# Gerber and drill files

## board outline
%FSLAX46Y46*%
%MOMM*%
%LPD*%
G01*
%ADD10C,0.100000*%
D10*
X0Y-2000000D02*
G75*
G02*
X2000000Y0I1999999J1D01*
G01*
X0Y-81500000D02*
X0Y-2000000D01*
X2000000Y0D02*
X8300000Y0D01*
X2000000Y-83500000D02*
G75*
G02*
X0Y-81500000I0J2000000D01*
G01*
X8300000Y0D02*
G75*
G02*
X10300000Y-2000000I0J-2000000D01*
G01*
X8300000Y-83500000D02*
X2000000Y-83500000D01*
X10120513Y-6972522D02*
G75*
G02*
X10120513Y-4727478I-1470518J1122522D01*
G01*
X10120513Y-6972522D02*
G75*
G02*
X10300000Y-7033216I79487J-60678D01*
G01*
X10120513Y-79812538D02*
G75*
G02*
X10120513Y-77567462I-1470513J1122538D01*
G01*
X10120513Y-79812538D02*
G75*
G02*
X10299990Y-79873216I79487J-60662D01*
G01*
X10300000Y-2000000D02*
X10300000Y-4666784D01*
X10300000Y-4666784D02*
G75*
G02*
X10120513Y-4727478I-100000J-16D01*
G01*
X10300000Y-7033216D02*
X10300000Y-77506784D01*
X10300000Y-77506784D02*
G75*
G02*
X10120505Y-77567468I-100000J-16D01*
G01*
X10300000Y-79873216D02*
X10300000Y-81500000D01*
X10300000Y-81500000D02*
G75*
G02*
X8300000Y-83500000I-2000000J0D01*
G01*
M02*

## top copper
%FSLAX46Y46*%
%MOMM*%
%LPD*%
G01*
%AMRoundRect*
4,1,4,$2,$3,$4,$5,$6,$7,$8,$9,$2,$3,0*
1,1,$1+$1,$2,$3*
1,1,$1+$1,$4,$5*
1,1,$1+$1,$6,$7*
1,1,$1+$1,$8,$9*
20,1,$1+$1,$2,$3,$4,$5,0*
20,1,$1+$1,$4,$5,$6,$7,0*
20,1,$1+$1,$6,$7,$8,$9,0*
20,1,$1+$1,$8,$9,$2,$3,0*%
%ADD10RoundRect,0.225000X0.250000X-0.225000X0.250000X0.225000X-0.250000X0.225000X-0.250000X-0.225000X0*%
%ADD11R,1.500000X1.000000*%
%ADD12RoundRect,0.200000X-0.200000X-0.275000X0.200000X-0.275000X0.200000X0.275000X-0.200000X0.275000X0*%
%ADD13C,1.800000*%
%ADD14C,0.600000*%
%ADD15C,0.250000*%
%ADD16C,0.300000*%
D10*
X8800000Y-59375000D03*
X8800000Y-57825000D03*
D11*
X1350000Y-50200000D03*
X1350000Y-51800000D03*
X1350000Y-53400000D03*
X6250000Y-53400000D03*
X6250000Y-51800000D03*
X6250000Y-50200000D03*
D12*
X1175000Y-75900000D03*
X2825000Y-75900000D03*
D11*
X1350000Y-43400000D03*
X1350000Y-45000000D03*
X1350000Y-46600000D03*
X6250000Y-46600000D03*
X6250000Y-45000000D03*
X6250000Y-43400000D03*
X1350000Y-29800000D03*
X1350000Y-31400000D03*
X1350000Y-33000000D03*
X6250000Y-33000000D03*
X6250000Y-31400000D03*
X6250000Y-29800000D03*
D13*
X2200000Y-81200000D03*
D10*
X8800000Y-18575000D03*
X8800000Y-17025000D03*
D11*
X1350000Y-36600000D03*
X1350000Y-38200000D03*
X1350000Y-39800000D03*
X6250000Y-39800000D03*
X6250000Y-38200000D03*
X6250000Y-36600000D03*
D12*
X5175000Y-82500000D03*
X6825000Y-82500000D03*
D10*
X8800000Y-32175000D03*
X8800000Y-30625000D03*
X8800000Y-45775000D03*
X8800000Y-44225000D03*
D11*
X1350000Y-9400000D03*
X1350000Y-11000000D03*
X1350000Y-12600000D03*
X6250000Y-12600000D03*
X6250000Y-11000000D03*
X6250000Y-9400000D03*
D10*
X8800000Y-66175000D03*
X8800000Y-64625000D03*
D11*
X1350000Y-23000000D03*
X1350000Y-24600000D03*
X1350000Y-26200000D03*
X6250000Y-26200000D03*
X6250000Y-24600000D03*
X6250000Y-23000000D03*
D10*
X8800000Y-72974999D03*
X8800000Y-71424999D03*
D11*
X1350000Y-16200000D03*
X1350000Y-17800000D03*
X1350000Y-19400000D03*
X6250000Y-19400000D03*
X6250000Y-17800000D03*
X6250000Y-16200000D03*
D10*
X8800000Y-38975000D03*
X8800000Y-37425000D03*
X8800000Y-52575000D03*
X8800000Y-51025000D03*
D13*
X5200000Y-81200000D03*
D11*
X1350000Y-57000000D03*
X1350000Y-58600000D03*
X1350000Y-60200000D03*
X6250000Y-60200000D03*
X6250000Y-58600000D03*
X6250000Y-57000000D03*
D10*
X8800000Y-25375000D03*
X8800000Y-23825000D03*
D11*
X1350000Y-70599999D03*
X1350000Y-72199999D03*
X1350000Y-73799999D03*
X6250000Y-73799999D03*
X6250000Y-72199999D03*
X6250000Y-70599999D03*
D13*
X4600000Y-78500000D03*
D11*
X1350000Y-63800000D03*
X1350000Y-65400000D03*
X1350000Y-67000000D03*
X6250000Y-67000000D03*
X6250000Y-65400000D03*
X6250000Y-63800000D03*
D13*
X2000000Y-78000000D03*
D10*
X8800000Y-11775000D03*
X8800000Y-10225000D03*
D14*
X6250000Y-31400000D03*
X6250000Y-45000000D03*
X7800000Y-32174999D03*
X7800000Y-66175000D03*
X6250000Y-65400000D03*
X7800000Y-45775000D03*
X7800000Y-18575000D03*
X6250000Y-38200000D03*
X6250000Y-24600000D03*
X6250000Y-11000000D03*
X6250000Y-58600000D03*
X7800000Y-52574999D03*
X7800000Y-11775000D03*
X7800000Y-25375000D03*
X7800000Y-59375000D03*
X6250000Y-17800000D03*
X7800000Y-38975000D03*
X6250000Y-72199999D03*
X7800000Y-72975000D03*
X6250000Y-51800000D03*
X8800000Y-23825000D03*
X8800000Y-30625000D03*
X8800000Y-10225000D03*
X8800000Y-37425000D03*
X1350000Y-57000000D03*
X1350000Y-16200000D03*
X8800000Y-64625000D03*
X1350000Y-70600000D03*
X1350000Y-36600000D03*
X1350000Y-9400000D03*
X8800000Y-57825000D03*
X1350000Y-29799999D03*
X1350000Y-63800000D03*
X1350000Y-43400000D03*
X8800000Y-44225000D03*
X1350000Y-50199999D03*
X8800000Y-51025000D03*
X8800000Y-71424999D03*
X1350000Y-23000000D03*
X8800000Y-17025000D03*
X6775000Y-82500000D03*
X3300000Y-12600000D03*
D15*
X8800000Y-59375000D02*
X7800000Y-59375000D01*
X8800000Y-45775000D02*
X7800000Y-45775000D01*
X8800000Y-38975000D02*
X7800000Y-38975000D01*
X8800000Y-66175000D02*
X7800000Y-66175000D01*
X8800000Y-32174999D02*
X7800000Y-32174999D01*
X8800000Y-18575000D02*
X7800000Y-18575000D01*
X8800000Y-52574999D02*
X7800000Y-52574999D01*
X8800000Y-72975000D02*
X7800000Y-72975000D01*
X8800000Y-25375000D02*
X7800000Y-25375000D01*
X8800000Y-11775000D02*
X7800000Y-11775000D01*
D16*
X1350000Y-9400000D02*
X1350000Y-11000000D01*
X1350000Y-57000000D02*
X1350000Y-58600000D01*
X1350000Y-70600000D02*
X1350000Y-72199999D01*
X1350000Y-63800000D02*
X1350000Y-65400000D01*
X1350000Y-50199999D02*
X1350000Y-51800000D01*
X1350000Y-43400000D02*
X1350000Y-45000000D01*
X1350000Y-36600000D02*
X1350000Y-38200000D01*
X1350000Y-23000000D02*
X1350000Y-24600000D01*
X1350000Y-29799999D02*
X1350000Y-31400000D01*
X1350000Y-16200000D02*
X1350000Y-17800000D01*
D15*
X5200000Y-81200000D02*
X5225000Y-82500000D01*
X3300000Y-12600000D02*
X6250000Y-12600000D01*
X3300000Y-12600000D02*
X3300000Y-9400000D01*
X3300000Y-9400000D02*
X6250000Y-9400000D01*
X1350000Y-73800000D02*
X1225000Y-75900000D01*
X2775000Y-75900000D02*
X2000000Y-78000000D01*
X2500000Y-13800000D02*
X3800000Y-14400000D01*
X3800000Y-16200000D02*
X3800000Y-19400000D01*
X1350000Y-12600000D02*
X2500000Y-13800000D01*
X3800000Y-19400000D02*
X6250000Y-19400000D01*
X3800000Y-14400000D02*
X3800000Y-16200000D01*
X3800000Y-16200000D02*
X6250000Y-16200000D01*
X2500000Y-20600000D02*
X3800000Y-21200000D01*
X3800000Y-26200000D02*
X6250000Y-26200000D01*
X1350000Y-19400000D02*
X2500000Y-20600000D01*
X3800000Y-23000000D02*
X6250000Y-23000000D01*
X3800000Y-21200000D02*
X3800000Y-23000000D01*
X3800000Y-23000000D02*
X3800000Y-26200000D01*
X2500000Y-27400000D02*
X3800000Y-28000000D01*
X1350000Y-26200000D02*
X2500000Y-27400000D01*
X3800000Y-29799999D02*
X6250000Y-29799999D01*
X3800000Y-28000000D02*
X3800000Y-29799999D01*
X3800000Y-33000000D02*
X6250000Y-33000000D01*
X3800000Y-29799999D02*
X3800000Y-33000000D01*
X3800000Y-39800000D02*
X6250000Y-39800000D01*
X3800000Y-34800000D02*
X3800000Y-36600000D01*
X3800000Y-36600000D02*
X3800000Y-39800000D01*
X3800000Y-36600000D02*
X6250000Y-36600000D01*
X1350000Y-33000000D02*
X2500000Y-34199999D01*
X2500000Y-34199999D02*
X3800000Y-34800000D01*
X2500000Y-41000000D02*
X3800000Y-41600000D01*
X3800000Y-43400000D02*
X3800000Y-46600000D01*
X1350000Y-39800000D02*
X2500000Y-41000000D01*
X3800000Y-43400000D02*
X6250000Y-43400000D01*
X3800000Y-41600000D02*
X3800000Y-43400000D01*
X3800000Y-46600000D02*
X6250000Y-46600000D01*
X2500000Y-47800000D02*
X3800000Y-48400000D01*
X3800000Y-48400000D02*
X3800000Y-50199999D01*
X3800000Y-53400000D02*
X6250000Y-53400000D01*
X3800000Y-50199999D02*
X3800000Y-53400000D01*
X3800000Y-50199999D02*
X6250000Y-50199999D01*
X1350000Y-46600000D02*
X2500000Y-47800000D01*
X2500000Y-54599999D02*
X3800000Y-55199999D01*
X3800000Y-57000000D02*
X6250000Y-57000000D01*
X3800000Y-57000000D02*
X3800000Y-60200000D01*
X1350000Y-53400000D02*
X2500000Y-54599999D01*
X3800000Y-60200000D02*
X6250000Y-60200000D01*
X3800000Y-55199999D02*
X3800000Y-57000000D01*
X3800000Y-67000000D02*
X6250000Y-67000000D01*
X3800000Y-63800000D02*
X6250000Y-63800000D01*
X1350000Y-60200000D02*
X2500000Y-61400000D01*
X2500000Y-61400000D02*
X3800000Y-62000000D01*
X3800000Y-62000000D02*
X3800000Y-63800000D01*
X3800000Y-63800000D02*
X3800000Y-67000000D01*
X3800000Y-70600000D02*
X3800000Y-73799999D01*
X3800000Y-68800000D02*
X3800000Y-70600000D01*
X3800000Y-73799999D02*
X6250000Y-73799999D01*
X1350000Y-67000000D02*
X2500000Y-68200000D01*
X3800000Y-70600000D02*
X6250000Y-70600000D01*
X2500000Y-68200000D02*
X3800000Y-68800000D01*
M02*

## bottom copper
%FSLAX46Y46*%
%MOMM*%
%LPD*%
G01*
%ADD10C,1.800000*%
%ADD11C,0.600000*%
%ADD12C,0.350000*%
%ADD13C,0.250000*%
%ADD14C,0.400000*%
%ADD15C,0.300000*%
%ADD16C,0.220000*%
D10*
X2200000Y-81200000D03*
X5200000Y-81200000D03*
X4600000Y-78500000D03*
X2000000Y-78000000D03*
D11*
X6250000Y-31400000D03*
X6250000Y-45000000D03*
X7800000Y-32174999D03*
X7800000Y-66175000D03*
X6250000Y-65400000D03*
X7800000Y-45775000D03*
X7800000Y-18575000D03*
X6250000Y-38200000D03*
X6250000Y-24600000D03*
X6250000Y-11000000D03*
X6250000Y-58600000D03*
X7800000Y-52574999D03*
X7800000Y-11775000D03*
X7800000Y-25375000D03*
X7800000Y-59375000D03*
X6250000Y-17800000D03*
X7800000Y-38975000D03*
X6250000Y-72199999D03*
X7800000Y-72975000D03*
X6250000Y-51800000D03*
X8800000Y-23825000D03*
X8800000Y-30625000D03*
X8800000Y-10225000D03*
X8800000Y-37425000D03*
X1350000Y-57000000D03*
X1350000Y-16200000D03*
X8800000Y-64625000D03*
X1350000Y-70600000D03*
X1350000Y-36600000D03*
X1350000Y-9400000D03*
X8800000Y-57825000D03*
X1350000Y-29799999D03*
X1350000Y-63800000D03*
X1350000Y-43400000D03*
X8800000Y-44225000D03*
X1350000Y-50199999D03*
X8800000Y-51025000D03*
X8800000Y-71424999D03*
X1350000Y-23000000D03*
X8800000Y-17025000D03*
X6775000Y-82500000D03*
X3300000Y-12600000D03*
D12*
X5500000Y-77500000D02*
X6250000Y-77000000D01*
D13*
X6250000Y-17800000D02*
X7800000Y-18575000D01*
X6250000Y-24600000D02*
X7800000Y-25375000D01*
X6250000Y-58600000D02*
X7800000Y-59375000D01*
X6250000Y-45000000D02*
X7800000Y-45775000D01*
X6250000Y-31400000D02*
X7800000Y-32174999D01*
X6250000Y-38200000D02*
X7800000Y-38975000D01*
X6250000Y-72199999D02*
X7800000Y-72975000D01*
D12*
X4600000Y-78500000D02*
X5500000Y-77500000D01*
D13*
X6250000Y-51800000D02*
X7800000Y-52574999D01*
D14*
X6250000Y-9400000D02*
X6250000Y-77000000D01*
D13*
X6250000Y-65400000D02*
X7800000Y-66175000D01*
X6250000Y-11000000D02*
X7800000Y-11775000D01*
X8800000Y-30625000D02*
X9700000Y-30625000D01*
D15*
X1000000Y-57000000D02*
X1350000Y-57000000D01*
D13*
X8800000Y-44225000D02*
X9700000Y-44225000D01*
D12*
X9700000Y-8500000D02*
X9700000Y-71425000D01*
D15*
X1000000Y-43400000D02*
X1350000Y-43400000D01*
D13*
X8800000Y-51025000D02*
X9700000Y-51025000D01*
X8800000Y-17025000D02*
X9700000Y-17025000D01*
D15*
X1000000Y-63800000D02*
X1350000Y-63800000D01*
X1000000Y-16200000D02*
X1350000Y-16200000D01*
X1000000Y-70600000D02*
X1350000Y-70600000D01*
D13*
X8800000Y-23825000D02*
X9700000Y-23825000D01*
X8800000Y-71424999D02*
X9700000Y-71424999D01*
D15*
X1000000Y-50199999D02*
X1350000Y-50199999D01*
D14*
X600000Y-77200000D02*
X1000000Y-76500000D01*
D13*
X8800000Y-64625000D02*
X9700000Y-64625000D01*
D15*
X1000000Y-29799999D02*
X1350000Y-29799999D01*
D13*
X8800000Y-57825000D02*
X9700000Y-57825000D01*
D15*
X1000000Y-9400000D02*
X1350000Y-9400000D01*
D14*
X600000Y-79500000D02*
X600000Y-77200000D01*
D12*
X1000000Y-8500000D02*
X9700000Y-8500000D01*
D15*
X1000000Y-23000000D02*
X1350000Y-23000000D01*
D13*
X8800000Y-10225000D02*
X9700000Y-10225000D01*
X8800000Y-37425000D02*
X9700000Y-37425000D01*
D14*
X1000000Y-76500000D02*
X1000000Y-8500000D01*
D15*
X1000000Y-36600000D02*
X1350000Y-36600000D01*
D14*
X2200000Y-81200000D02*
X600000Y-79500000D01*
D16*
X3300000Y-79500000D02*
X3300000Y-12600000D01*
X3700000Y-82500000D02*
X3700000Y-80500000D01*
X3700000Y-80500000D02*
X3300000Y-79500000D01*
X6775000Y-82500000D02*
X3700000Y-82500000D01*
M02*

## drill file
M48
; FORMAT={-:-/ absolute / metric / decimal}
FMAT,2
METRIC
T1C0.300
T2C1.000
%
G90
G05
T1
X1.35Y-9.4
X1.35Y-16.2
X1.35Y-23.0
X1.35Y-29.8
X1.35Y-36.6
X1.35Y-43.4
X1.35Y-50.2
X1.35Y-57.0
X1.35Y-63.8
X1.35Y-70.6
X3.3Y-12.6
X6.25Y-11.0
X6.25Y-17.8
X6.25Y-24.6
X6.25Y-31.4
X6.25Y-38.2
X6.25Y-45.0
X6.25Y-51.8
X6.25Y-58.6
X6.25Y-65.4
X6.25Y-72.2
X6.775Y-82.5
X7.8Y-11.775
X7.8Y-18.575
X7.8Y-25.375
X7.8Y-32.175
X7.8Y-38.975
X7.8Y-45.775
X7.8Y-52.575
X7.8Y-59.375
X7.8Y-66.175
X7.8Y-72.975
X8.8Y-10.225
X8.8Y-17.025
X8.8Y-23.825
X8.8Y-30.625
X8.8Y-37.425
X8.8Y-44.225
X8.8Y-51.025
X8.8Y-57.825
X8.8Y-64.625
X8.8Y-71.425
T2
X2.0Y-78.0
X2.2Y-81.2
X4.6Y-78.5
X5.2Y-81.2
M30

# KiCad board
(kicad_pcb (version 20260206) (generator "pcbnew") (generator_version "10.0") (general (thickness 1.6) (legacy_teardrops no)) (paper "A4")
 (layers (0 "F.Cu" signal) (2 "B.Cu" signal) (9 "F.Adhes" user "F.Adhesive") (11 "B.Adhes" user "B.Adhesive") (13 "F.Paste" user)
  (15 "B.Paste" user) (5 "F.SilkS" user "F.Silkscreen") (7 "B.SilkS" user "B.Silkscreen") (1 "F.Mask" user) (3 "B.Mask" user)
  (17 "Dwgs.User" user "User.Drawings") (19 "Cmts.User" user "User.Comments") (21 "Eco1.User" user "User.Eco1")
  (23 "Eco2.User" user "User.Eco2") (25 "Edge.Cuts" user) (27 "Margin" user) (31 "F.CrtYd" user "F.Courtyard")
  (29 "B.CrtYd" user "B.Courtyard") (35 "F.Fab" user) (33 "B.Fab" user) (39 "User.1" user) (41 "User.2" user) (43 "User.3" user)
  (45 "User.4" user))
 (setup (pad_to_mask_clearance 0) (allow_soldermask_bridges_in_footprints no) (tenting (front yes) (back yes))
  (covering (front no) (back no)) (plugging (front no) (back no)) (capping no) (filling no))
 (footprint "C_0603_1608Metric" (layer "F.Cu") (at 8.8 58.6 90)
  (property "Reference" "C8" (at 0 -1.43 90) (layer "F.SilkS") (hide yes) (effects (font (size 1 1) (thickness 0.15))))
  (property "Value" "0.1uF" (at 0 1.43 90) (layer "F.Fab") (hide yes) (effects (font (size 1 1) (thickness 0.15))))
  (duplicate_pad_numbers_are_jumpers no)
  (pad "1" smd roundrect (at -0.775 0 90) (size 0.9 0.95) (layers "F.Cu" "F.Mask" "F.Paste") (roundrect_rratio 0.25) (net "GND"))
  (pad "2" smd roundrect (at 0.775 0 90) (size 0.9 0.95) (layers "F.Cu" "F.Mask" "F.Paste") (roundrect_rratio 0.25) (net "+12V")))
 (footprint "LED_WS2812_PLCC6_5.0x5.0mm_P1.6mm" (layer "F.Cu") (at 3.8 51.8)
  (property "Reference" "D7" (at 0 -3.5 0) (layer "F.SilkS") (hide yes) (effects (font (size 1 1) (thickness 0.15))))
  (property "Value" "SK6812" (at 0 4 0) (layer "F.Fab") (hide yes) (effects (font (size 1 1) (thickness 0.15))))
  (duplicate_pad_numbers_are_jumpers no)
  (pad "1" smd rect (at -2.45 -1.6) (size 1.5 1) (layers "F.Cu" "F.Mask" "F.Paste") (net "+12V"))
  (pad "2" smd rect (at -2.45 0) (size 1.5 1) (layers "F.Cu" "F.Mask" "F.Paste") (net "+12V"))
  (pad "3" smd rect (at -2.45 1.6) (size 1.5 1) (layers "F.Cu" "F.Mask" "F.Paste") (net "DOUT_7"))
  (pad "4" smd rect (at 2.45 1.6) (size 1.5 1) (layers "F.Cu" "F.Mask" "F.Paste") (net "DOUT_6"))
  (pad "5" smd rect (at 2.45 0) (size 1.5 1) (layers "F.Cu" "F.Mask" "F.Paste") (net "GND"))
  (pad "6" smd rect (at 2.45 -1.6) (size 1.5 1) (layers "F.Cu" "F.Mask" "F.Paste") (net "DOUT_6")))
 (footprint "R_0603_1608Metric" (layer "F.Cu") (at 2 75.9)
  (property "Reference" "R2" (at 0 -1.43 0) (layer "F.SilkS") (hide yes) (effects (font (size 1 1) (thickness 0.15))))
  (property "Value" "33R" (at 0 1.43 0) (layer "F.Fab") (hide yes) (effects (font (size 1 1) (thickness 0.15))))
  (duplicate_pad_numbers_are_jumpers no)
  (pad "1" smd roundrect (at -0.825 0) (size 0.8 0.95) (layers "F.Cu" "F.Mask" "F.Paste") (roundrect_rratio 0.25) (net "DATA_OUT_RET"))
  (pad "2" smd roundrect (at 0.825 0) (size 0.8 0.95) (layers "F.Cu" "F.Mask" "F.Paste") (roundrect_rratio 0.25) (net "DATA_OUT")))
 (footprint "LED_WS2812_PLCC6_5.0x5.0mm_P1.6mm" (layer "F.Cu") (at 3.8 45)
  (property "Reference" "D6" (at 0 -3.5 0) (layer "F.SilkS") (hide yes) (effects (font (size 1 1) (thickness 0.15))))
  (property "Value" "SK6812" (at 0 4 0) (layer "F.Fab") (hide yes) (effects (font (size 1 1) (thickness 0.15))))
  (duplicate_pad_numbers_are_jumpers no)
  (pad "1" smd rect (at -2.45 -1.6) (size 1.5 1) (layers "F.Cu" "F.Mask" "F.Paste") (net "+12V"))
  (pad "2" smd rect (at -2.45 0) (size 1.5 1) (layers "F.Cu" "F.Mask" "F.Paste") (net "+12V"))
  (pad "3" smd rect (at -2.45 1.6) (size 1.5 1) (layers "F.Cu" "F.Mask" "F.Paste") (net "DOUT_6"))
  (pad "4" smd rect (at 2.45 1.6) (size 1.5 1) (layers "F.Cu" "F.Mask" "F.Paste") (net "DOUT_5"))
  (pad "5" smd rect (at 2.45 0) (size 1.5 1) (layers "F.Cu" "F.Mask" "F.Paste") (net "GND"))
  (pad "6" smd rect (at 2.45 -1.6) (size 1.5 1) (layers "F.Cu" "F.Mask" "F.Paste") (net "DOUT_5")))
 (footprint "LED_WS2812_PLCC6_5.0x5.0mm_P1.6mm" (layer "F.Cu") (at 3.8 31.4)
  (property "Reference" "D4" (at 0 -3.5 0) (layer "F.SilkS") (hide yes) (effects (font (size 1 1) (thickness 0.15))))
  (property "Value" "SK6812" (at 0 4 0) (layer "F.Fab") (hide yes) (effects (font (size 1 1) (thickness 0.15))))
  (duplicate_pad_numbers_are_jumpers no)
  (pad "1" smd rect (at -2.45 -1.6) (size 1.5 1) (layers "F.Cu" "F.Mask" "F.Paste") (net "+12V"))
  (pad "2" smd rect (at -2.45 0) (size 1.5 1) (layers "F.Cu" "F.Mask" "F.Paste") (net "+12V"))
  (pad "3" smd rect (at -2.45 1.6) (size 1.5 1) (layers "F.Cu" "F.Mask" "F.Paste") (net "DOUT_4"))
  (pad "4" smd rect (at 2.45 1.6) (size 1.5 1) (layers "F.Cu" "F.Mask" "F.Paste") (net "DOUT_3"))
  (pad "5" smd rect (at 2.45 0) (size 1.5 1) (layers "F.Cu" "F.Mask" "F.Paste") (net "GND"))
  (pad "6" smd rect (at 2.45 -1.6) (size 1.5 1) (layers "F.Cu" "F.Mask" "F.Paste") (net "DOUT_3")))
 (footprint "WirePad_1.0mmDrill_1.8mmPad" (layer "F.Cu") (at 2.2 81.2)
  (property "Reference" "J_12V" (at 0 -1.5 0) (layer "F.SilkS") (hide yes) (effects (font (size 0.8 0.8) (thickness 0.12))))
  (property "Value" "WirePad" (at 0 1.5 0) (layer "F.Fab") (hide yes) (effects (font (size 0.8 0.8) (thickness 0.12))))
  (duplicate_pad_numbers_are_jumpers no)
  (pad "1" thru_hole circle (at 0 0) (size 1.8 1.8) (drill 1) (layers "*.Cu" "*.Mask") (remove_unused_layers no) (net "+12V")))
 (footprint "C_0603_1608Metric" (layer "F.Cu") (at 8.8 17.8 90)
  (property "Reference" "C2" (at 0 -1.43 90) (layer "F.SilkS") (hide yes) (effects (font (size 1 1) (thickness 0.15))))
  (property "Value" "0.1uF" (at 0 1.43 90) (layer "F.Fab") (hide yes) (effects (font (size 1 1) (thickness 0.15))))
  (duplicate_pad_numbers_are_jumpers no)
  (pad "1" smd roundrect (at -0.775 0 90) (size 0.9 0.95) (layers "F.Cu" "F.Mask" "F.Paste") (roundrect_rratio 0.25) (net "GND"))
  (pad "2" smd roundrect (at 0.775 0 90) (size 0.9 0.95) (layers "F.Cu" "F.Mask" "F.Paste") (roundrect_rratio 0.25) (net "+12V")))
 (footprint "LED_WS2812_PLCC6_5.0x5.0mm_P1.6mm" (layer "F.Cu") (at 3.8 38.2)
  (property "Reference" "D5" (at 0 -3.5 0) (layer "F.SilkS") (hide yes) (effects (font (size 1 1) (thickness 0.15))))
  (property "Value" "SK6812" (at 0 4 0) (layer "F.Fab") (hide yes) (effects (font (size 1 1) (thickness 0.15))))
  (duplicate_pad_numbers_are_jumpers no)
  (pad "1" smd rect (at -2.45 -1.6) (size 1.5 1) (layers "F.Cu" "F.Mask" "F.Paste") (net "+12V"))
  (pad "2" smd rect (at -2.45 0) (size 1.5 1) (layers "F.Cu" "F.Mask" "F.Paste") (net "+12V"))
  (pad "3" smd rect (at -2.45 1.6) (size 1.5 1) (layers "F.Cu" "F.Mask" "F.Paste") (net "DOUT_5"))
  (pad "4" smd rect (at 2.45 1.6) (size 1.5 1) (layers "F.Cu" "F.Mask" "F.Paste") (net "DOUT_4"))
  (pad "5" smd rect (at 2.45 0) (size 1.5 1) (layers "F.Cu" "F.Mask" "F.Paste") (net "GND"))
  (pad "6" smd rect (at 2.45 -1.6) (size 1.5 1) (layers "F.Cu" "F.Mask" "F.Paste") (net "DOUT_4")))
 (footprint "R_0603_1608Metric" (layer "F.Cu") (at 6 82.5)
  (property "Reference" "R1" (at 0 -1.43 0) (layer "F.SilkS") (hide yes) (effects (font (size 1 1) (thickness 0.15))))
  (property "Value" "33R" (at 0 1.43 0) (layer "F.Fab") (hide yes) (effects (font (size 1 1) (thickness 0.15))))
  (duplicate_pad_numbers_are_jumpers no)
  (pad "1" smd roundrect (at -0.825 0) (size 0.8 0.95) (layers "F.Cu" "F.Mask" "F.Paste") (roundrect_rratio 0.25) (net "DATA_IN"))
  (pad "2" smd roundrect (at 0.825 0) (size 0.8 0.95) (layers "F.Cu" "F.Mask" "F.Paste") (roundrect_rratio 0.25) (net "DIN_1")))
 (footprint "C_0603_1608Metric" (layer "F.Cu") (at 8.8 31.4 90)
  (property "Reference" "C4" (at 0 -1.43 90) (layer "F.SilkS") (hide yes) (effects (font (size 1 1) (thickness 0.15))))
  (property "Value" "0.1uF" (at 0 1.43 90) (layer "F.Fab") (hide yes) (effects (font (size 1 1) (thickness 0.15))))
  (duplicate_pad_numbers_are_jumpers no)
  (pad "1" smd roundrect (at -0.775 0 90) (size 0.9 0.95) (layers "F.Cu" "F.Mask" "F.Paste") (roundrect_rratio 0.25) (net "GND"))
  (pad "2" smd roundrect (at 0.775 0 90) (size 0.9 0.95) (layers "F.Cu" "F.Mask" "F.Paste") (roundrect_rratio 0.25) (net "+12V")))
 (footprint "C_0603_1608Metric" (layer "F.Cu") (at 8.8 45 90)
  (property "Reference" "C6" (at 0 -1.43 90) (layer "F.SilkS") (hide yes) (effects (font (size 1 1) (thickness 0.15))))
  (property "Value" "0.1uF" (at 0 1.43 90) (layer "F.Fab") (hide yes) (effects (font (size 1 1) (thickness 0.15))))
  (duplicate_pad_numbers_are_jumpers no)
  (pad "1" smd roundrect (at -0.775 0 90) (size 0.9 0.95) (layers "F.Cu" "F.Mask" "F.Paste") (roundrect_rratio 0.25) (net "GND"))
  (pad "2" smd roundrect (at 0.775 0 90) (size 0.9 0.95) (layers "F.Cu" "F.Mask" "F.Paste") (roundrect_rratio 0.25) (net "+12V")))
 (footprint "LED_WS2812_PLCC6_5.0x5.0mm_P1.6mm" (layer "F.Cu") (at 3.8 11)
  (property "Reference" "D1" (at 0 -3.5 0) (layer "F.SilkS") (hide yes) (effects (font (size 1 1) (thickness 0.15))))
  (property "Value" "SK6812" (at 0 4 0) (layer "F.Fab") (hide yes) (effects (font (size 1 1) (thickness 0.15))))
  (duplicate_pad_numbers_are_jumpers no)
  (pad "1" smd rect (at -2.45 -1.6) (size 1.5 1) (layers "F.Cu" "F.Mask" "F.Paste") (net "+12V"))
  (pad "2" smd rect (at -2.45 0) (size 1.5 1) (layers "F.Cu" "F.Mask" "F.Paste") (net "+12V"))
  (pad "3" smd rect (at -2.45 1.6) (size 1.5 1) (layers "F.Cu" "F.Mask" "F.Paste") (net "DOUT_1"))
  (pad "4" smd rect (at 2.45 1.6) (size 1.5 1) (layers "F.Cu" "F.Mask" "F.Paste") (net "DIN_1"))
  (pad "5" smd rect (at 2.45 0) (size 1.5 1) (layers "F.Cu" "F.Mask" "F.Paste") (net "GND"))
  (pad "6" smd rect (at 2.45 -1.6) (size 1.5 1) (layers "F.Cu" "F.Mask" "F.Paste") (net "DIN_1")))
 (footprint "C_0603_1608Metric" (layer "F.Cu") (at 8.8 65.4 90)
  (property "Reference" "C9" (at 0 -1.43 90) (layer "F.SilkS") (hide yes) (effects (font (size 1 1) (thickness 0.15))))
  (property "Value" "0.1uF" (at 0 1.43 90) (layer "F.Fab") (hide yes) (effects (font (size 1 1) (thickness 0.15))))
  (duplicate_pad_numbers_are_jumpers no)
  (pad "1" smd roundrect (at -0.775 0 90) (size 0.9 0.95) (layers "F.Cu" "F.Mask" "F.Paste") (roundrect_rratio 0.25) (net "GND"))
  (pad "2" smd roundrect (at 0.775 0 90) (size 0.9 0.95) (layers "F.Cu" "F.Mask" "F.Paste") (roundrect_rratio 0.25) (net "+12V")))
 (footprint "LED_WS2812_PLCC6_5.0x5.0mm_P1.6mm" (layer "F.Cu") (at 3.8 24.6)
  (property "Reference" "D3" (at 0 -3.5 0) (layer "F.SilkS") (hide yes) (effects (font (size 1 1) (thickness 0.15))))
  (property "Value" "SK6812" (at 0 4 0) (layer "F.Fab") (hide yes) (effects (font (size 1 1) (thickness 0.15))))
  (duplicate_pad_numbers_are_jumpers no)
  (pad "1" smd rect (at -2.45 -1.6) (size 1.5 1) (layers "F.Cu" "F.Mask" "F.Paste") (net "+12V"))
  (pad "2" smd rect (at -2.45 0) (size 1.5 1) (layers "F.Cu" "F.Mask" "F.Paste") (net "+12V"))
  (pad "3" smd rect (at -2.45 1.6) (size 1.5 1) (layers "F.Cu" "F.Mask" "F.Paste") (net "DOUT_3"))
  (pad "4" smd rect (at 2.45 1.6) (size 1.5 1) (layers "F.Cu" "F.Mask" "F.Paste") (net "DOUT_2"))
  (pad "5" smd rect (at 2.45 0) (size 1.5 1) (layers "F.Cu" "F.Mask" "F.Paste") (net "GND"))
  (pad "6" smd rect (at 2.45 -1.6) (size 1.5 1) (layers "F.Cu" "F.Mask" "F.Paste") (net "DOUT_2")))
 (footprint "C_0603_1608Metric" (layer "F.Cu") (at 8.8 72.199999 90)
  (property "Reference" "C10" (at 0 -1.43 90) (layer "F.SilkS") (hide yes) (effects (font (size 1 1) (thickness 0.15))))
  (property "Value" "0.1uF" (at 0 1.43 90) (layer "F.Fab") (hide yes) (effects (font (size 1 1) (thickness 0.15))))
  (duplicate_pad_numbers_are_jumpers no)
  (pad "1" smd roundrect (at -0.775 0 90) (size 0.9 0.95) (layers "F.Cu" "F.Mask" "F.Paste") (roundrect_rratio 0.25) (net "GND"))
  (pad "2" smd roundrect (at 0.775 0 90) (size 0.9 0.95) (layers "F.Cu" "F.Mask" "F.Paste") (roundrect_rratio 0.25) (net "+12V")))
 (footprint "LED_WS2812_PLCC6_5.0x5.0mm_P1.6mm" (layer "F.Cu") (at 3.8 17.8)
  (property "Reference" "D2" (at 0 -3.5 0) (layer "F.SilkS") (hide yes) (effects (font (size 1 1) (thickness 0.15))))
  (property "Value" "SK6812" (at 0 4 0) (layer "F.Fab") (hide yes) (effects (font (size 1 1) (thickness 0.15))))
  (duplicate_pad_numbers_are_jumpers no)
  (pad "1" smd rect (at -2.45 -1.6) (size 1.5 1) (layers "F.Cu" "F.Mask" "F.Paste") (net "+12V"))
  (pad "2" smd rect (at -2.45 0) (size 1.5 1) (layers "F.Cu" "F.Mask" "F.Paste") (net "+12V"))
  (pad "3" smd rect (at -2.45 1.6) (size 1.5 1) (layers "F.Cu" "F.Mask" "F.Paste") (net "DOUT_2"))
  (pad "4" smd rect (at 2.45 1.6) (size 1.5 1) (layers "F.Cu" "F.Mask" "F.Paste") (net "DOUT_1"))
  (pad "5" smd rect (at 2.45 0) (size 1.5 1) (layers "F.Cu" "F.Mask" "F.Paste") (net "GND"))
  (pad "6" smd rect (at 2.45 -1.6) (size 1.5 1) (layers "F.Cu" "F.Mask" "F.Paste") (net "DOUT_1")))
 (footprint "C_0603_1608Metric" (layer "F.Cu") (at 8.8 38.2 90)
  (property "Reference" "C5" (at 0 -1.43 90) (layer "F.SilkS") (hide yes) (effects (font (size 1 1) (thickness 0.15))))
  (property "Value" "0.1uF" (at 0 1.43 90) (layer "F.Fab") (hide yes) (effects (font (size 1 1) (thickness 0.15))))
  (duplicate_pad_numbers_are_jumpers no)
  (pad "1" smd roundrect (at -0.775 0 90) (size 0.9 0.95) (layers "F.Cu" "F.Mask" "F.Paste") (roundrect_rratio 0.25) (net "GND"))
  (pad "2" smd roundrect (at 0.775 0 90) (size 0.9 0.95) (layers "F.Cu" "F.Mask" "F.Paste") (roundrect_rratio 0.25) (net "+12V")))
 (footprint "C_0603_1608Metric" (layer "F.Cu") (at 8.8 51.8 90)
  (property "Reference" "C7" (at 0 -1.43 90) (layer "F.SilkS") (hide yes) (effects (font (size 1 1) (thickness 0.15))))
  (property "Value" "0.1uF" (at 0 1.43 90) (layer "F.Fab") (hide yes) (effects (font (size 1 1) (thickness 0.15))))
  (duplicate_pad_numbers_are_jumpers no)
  (pad "1" smd roundrect (at -0.775 0 90) (size 0.9 0.95) (layers "F.Cu" "F.Mask" "F.Paste") (roundrect_rratio 0.25) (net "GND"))
  (pad "2" smd roundrect (at 0.775 0 90) (size 0.9 0.95) (layers "F.Cu" "F.Mask" "F.Paste") (roundrect_rratio 0.25) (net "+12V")))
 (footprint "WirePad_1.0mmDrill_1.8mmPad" (layer "F.Cu") (at 5.2 81.2)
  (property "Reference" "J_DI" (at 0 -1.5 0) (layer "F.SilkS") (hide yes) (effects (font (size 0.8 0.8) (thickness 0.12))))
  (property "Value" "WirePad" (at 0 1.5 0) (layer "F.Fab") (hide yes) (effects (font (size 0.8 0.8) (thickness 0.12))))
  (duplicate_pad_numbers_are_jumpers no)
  (pad "1" thru_hole circle (at 0 0) (size 1.8 1.8) (drill 1) (layers "*.Cu" "*.Mask") (remove_unused_layers no) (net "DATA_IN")))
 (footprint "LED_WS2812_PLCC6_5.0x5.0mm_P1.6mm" (layer "F.Cu") (at 3.8 58.6)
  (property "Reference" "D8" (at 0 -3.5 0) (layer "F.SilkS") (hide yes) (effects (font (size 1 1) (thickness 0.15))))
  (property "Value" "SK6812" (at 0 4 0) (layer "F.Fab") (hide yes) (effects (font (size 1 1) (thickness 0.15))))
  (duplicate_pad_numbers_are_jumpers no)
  (pad "1" smd rect (at -2.45 -1.6) (size 1.5 1) (layers "F.Cu" "F.Mask" "F.Paste") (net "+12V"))
  (pad "2" smd rect (at -2.45 0) (size 1.5 1) (layers "F.Cu" "F.Mask" "F.Paste") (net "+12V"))
  (pad "3" smd rect (at -2.45 1.6) (size 1.5 1) (layers "F.Cu" "F.Mask" "F.Paste") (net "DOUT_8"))
  (pad "4" smd rect (at 2.45 1.6) (size 1.5 1) (layers "F.Cu" "F.Mask" "F.Paste") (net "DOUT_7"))
  (pad "5" smd rect (at 2.45 0) (size 1.5 1) (layers "F.Cu" "F.Mask" "F.Paste") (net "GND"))
  (pad "6" smd rect (at 2.45 -1.6) (size 1.5 1) (layers "F.Cu" "F.Mask" "F.Paste") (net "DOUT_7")))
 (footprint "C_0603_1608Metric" (layer "F.Cu") (at 8.8 24.6 90)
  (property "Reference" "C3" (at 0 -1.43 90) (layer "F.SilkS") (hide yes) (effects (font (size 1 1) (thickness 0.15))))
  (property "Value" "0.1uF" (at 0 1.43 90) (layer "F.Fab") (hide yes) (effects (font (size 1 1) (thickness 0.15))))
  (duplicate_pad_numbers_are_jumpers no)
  (pad "1" smd roundrect (at -0.775 0 90) (size 0.9 0.95) (layers "F.Cu" "F.Mask" "F.Paste") (roundrect_rratio 0.25) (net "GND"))
  (pad "2" smd roundrect (at 0.775 0 90) (size 0.9 0.95) (layers "F.Cu" "F.Mask" "F.Paste") (roundrect_rratio 0.25) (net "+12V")))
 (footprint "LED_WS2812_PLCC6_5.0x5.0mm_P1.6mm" (layer "F.Cu") (at 3.8 72.199999)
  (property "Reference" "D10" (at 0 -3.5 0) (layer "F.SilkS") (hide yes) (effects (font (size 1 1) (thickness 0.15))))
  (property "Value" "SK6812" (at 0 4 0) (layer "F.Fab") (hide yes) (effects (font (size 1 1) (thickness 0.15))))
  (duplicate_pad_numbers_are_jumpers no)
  (pad "1" smd rect (at -2.45 -1.6) (size 1.5 1) (layers "F.Cu" "F.Mask" "F.Paste") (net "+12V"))
  (pad "2" smd rect (at -2.45 0) (size 1.5 1) (layers "F.Cu" "F.Mask" "F.Paste") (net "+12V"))
  (pad "3" smd rect (at -2.45 1.6) (size 1.5 1) (layers "F.Cu" "F.Mask" "F.Paste") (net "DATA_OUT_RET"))
  (pad "4" smd rect (at 2.45 1.6) (size 1.5 1) (layers "F.Cu" "F.Mask" "F.Paste") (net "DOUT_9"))
  (pad "5" smd rect (at 2.45 0) (size 1.5 1) (layers "F.Cu" "F.Mask" "F.Paste") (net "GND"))
  (pad "6" smd rect (at 2.45 -1.6) (size 1.5 1) (layers "F.Cu" "F.Mask" "F.Paste") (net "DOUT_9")))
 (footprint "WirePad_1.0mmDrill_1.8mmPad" (layer "F.Cu") (at 4.6 78.5)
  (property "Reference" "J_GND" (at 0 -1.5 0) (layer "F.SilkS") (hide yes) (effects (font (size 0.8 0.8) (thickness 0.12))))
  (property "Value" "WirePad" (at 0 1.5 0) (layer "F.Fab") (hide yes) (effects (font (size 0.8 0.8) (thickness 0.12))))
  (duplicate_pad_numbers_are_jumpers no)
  (pad "1" thru_hole circle (at 0 0) (size 1.8 1.8) (drill 1) (layers "*.Cu" "*.Mask") (remove_unused_layers no) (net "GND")))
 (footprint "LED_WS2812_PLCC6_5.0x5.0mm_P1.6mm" (layer "F.Cu") (at 3.8 65.4)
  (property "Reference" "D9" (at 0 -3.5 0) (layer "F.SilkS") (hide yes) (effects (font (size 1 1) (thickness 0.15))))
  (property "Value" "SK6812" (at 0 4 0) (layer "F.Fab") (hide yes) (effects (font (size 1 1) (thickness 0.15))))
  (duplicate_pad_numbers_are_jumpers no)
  (pad "1" smd rect (at -2.45 -1.6) (size 1.5 1) (layers "F.Cu" "F.Mask" "F.Paste") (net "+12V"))
  (pad "2" smd rect (at -2.45 0) (size 1.5 1) (layers "F.Cu" "F.Mask" "F.Paste") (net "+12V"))
  (pad "3" smd rect (at -2.45 1.6) (size 1.5 1) (layers "F.Cu" "F.Mask" "F.Paste") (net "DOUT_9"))
  (pad "4" smd rect (at 2.45 1.6) (size 1.5 1) (layers "F.Cu" "F.Mask" "F.Paste") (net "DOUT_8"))
  (pad "5" smd rect (at 2.45 0) (size 1.5 1) (layers "F.Cu" "F.Mask" "F.Paste") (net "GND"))
  (pad "6" smd rect (at 2.45 -1.6) (size 1.5 1) (layers "F.Cu" "F.Mask" "F.Paste") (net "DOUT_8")))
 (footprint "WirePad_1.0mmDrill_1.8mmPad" (layer "F.Cu") (at 2 78)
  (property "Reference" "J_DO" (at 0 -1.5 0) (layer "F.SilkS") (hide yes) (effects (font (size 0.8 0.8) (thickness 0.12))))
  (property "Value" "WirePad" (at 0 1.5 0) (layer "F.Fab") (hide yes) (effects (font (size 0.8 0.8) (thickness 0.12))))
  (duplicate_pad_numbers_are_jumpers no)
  (pad "1" thru_hole circle (at 0 0) (size 1.8 1.8) (drill 1) (layers "*.Cu" "*.Mask") (remove_unused_layers no) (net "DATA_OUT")))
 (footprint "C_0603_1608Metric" (layer "F.Cu") (at 8.8 11 90)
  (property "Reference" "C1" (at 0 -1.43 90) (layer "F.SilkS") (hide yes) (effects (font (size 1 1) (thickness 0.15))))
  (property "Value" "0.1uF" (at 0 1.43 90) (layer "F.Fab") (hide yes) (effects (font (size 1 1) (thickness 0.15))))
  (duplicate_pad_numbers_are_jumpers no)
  (pad "1" smd roundrect (at -0.775 0 90) (size 0.9 0.95) (layers "F.Cu" "F.Mask" "F.Paste") (roundrect_rratio 0.25) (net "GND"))
  (pad "2" smd roundrect (at 0.775 0 90) (size 0.9 0.95) (layers "F.Cu" "F.Mask" "F.Paste") (roundrect_rratio 0.25) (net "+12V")))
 (gr_arc (start 0 2) (mid 0.585786 0.585786) (end 2 0) (stroke (width 0.1) (type default)) (layer "Edge.Cuts"))
 (gr_line (start 0 81.5) (end 0 2) (stroke (width 0.1) (type default)) (layer "Edge.Cuts"))
 (gr_line (start 2 0) (end 8.3 0) (stroke (width 0.1) (type default)) (layer "Edge.Cuts"))
 (gr_arc (start 2 83.5) (mid 0.585786 82.914214) (end 0 81.5) (stroke (width 0.1) (type default)) (layer "Edge.Cuts"))
 (gr_arc (start 8.3 0) (mid 9.714214 0.585786) (end 10.3 2) (stroke (width 0.1) (type default)) (layer "Edge.Cuts"))
 (gr_line (start 8.3 83.5) (end 2 83.5) (stroke (width 0.1) (type default)) (layer "Edge.Cuts"))
 (gr_arc (start 10.120513 6.972522) (mid 6.800001 5.85) (end 10.120513 4.727478) (stroke (width 0.1) (type default)) (layer "Edge.Cuts"))
 (gr_arc (start 10.120513 6.972522) (mid 10.232025 6.938483) (end 10.3 7.033216) (stroke (width 0.1) (type default)) (layer "Edge.Cuts"))
 (gr_arc (start 10.120513 79.812538) (mid 6.8 78.69) (end 10.120513 77.567462) (stroke (width 0.1) (type default)) (layer "Edge.Cuts"))
 (gr_arc (start 10.120513 79.812538) (mid 10.232025 79.778483) (end 10.3 79.873216) (stroke (width 0.1) (type default)) (layer "Edge.Cuts"))
 (gr_line (start 10.3 2) (end 10.3 4.666784) (stroke (width 0.1) (type default)) (layer "Edge.Cuts"))
 (gr_arc (start 10.3 4.666784) (mid 10.232025 4.761517) (end 10.120513 4.727478) (stroke (width 0.1) (type default)) (layer "Edge.Cuts"))
 (gr_line (start 10.3 7.033216) (end 10.3 77.506784) (stroke (width 0.1) (type default)) (layer "Edge.Cuts"))
 (gr_arc (start 10.3 77.506784) (mid 10.232025 77.601517) (end 10.120513 77.567462) (stroke (width 0.1) (type default)) (layer "Edge.Cuts"))
 (gr_line (start 10.3 79.873216) (end 10.3 81.5) (stroke (width 0.1) (type default)) (layer "Edge.Cuts"))
 (gr_arc (start 10.3 81.5) (mid 9.714214 82.914214) (end 8.3 83.5) (stroke (width 0.1) (type default)) (layer "Edge.Cuts"))
 (segment (start 8.8 59.375) (end 7.8 59.375) (width 0.25) (layer "F.Cu") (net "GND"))
 (segment (start 8.8 45.775) (end 7.8 45.775) (width 0.25) (layer "F.Cu") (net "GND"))
 (segment (start 8.8 38.975) (end 7.8 38.975) (width 0.25) (layer "F.Cu") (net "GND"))
 (segment (start 8.8 66.175) (end 7.8 66.175) (width 0.25) (layer "F.Cu") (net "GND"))
 (segment (start 8.8 32.174999) (end 7.8 32.174999) (width 0.25) (layer "F.Cu") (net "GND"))
 (segment (start 8.8 18.575) (end 7.8 18.575) (width 0.25) (layer "F.Cu") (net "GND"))
 (segment (start 8.8 52.574999) (end 7.8 52.574999) (width 0.25) (layer "F.Cu") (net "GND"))
 (segment (start 8.8 72.975) (end 7.8 72.975) (width 0.25) (layer "F.Cu") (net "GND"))
 (segment (start 8.8 25.375) (end 7.8 25.375) (width 0.25) (layer "F.Cu") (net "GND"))
 (segment (start 8.8 11.775) (end 7.8 11.775) (width 0.25) (layer "F.Cu") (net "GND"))
 (via (at 6.25 31.4) (size 0.6) (drill 0.3) (layers "F.Cu" "B.Cu") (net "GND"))
 (via (at 6.25 45) (size 0.6) (drill 0.3) (layers "F.Cu" "B.Cu") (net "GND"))
 (via (at 7.8 32.174999) (size 0.6) (drill 0.3) (layers "F.Cu" "B.Cu") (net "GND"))
 (via (at 7.8 66.175) (size 0.6) (drill 0.3) (layers "F.Cu" "B.Cu") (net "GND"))
 (via (at 6.25 65.4) (size 0.6) (drill 0.3) (layers "F.Cu" "B.Cu") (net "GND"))
 (via (at 7.8 45.775) (size 0.6) (drill 0.3) (layers "F.Cu" "B.Cu") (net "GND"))
 (via (at 7.8 18.575) (size 0.6) (drill 0.3) (layers "F.Cu" "B.Cu") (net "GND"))
 (via (at 6.25 38.2) (size 0.6) (drill 0.3) (layers "F.Cu" "B.Cu") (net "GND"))
 (via (at 6.25 24.6) (size 0.6) (drill 0.3) (layers "F.Cu" "B.Cu") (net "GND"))
 (via (at 6.25 11) (size 0.6) (drill 0.3) (layers "F.Cu" "B.Cu") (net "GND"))
 (via (at 6.25 58.6) (size 0.6) (drill 0.3) (layers "F.Cu" "B.Cu") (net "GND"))
 (via (at 7.8 52.574999) (size 0.6) (drill 0.3) (layers "F.Cu" "B.Cu") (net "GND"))
 (via (at 7.8 11.775) (size 0.6) (drill 0.3) (layers "F.Cu" "B.Cu") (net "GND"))
 (via (at 7.8 25.375) (size 0.6) (drill 0.3) (layers "F.Cu" "B.Cu") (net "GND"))
 (via (at 7.8 59.375) (size 0.6) (drill 0.3) (layers "F.Cu" "B.Cu") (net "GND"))
 (via (at 6.25 17.8) (size 0.6) (drill 0.3) (layers "F.Cu" "B.Cu") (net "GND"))
 (via (at 7.8 38.975) (size 0.6) (drill 0.3) (layers "F.Cu" "B.Cu") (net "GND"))
 (via (at 6.25 72.199999) (size 0.6) (drill 0.3) (layers "F.Cu" "B.Cu") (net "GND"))
 (via (at 7.8 72.975) (size 0.6) (drill 0.3) (layers "F.Cu" "B.Cu") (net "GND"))
 (via (at 6.25 51.8) (size 0.6) (drill 0.3) (layers "F.Cu" "B.Cu") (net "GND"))
 (segment (start 5.5 77.5) (end 6.25 77) (width 0.35) (layer "B.Cu") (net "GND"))
 (segment (start 6.25 17.8) (end 7.8 18.575) (width 0.25) (layer "B.Cu") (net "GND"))
 (segment (start 6.25 24.6) (end 7.8 25.375) (width 0.25) (layer "B.Cu") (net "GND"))
 (segment (start 6.25 58.6) (end 7.8 59.375) (width 0.25) (layer "B.Cu") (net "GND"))
 (segment (start 6.25 45) (end 7.8 45.775) (width 0.25) (layer "B.Cu") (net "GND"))
 (segment (start 6.25 31.4) (end 7.8 32.174999) (width 0.25) (layer "B.Cu") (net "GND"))
 (segment (start 6.25 38.2) (end 7.8 38.975) (width 0.25) (layer "B.Cu") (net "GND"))
 (segment (start 6.25 72.199999) (end 7.8 72.975) (width 0.25) (layer "B.Cu") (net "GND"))
 (segment (start 4.6 78.5) (end 5.5 77.5) (width 0.35) (layer "B.Cu") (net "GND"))
 (segment (start 6.25 51.8) (end 7.8 52.574999) (width 0.25) (layer "B.Cu") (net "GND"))
 (segment (start 6.25 9.4) (end 6.25 77) (width 0.4) (layer "B.Cu") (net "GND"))
 (segment (start 6.25 65.4) (end 7.8 66.175) (width 0.25) (layer "B.Cu") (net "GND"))
 (segment (start 6.25 11) (end 7.8 11.775) (width 0.25) (layer "B.Cu") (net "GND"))
 (segment (start 1.35 9.4) (end 1.35 11) (width 0.3) (layer "F.Cu") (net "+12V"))
 (segment (start 1.35 57) (end 1.35 58.6) (width 0.3) (layer "F.Cu") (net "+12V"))
 (segment (start 1.35 70.6) (end 1.35 72.199999) (width 0.3) (layer "F.Cu") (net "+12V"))
 (segment (start 1.35 63.8) (end 1.35 65.4) (width 0.3) (layer "F.Cu") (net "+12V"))
 (segment (start 1.35 50.199999) (end 1.35 51.8) (width 0.3) (layer "F.Cu") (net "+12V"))
 (segment (start 1.35 43.4) (end 1.35 45) (width 0.3) (layer "F.Cu") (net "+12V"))
 (segment (start 1.35 36.6) (end 1.35 38.2) (width 0.3) (layer "F.Cu") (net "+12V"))
 (segment (start 1.35 23) (end 1.35 24.6) (width 0.3) (layer "F.Cu") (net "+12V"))
 (segment (start 1.35 29.799999) (end 1.35 31.4) (width 0.3) (layer "F.Cu") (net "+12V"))
 (segment (start 1.35 16.2) (end 1.35 17.8) (width 0.3) (layer "F.Cu") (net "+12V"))
 (via (at 8.8 23.825) (size 0.6) (drill 0.3) (layers "F.Cu" "B.Cu") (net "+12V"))
 (via (at 8.8 30.625) (size 0.6) (drill 0.3) (layers "F.Cu" "B.Cu") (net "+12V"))
 (via (at 8.8 10.225) (size 0.6) (drill 0.3) (layers "F.Cu" "B.Cu") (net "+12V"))
 (via (at 8.8 37.425) (size 0.6) (drill 0.3) (layers "F.Cu" "B.Cu") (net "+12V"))
 (via (at 1.35 57) (size 0.6) (drill 0.3) (layers "F.Cu" "B.Cu") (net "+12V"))
 (via (at 1.35 16.2) (size 0.6) (drill 0.3) (layers "F.Cu" "B.Cu") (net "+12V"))
 (via (at 8.8 64.625) (size 0.6) (drill 0.3) (layers "F.Cu" "B.Cu") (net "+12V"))
 (via (at 1.35 70.6) (size 0.6) (drill 0.3) (layers "F.Cu" "B.Cu") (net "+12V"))
 (via (at 1.35 36.6) (size 0.6) (drill 0.3) (layers "F.Cu" "B.Cu") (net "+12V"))
 (via (at 1.35 9.4) (size 0.6) (drill 0.3) (layers "F.Cu" "B.Cu") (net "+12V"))
 (via (at 8.8 57.825) (size 0.6) (drill 0.3) (layers "F.Cu" "B.Cu") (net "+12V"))
 (via (at 1.35 29.799999) (size 0.6) (drill 0.3) (layers "F.Cu" "B.Cu") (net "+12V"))
 (via (at 1.35 63.8) (size 0.6) (drill 0.3) (layers "F.Cu" "B.Cu") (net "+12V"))
 (via (at 1.35 43.4) (size 0.6) (drill 0.3) (layers "F.Cu" "B.Cu") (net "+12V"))
 (via (at 8.8 44.225) (size 0.6) (drill 0.3) (layers "F.Cu" "B.Cu") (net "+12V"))
 (via (at 1.35 50.199999) (size 0.6) (drill 0.3) (layers "F.Cu" "B.Cu") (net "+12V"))
 (via (at 8.8 51.025) (size 0.6) (drill 0.3) (layers "F.Cu" "B.Cu") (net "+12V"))
 (via (at 8.8 71.424999) (size 0.6) (drill 0.3) (layers "F.Cu" "B.Cu") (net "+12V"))
 (via (at 1.35 23) (size 0.6) (drill 0.3) (layers "F.Cu" "B.Cu") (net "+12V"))
 (via (at 8.8 17.025) (size 0.6) (drill 0.3) (layers "F.Cu" "B.Cu") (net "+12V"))
 (segment (start 8.8 30.625) (end 9.7 30.625) (width 0.25) (layer "B.Cu") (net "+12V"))
 (segment (start 1 57) (end 1.35 57) (width 0.3) (layer "B.Cu") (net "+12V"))
 (segment (start 8.8 44.225) (end 9.7 44.225) (width 0.25) (layer "B.Cu") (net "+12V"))
 (segment (start 9.7 8.5) (end 9.7 71.425) (width 0.35) (layer "B.Cu") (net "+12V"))
 (segment (start 1 43.4) (end 1.35 43.4) (width 0.3) (layer "B.Cu") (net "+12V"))
 (segment (start 8.8 51.025) (end 9.7 51.025) (width 0.25) (layer "B.Cu") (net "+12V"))
 (segment (start 8.8 17.025) (end 9.7 17.025) (width 0.25) (layer "B.Cu") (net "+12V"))
 (segment (start 1 63.8) (end 1.35 63.8) (width 0.3) (layer "B.Cu") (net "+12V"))
 (segment (start 1 16.2) (end 1.35 16.2) (width 0.3) (layer "B.Cu") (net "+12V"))
 (segment (start 1 70.6) (end 1.35 70.6) (width 0.3) (layer "B.Cu") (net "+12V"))
 (segment (start 8.8 23.825) (end 9.7 23.825) (width 0.25) (layer "B.Cu") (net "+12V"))
 (segment (start 8.8 71.424999) (end 9.7 71.424999) (width 0.25) (layer "B.Cu") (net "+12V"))
 (segment (start 1 50.199999) (end 1.35 50.199999) (width 0.3) (layer "B.Cu") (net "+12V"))
 (segment (start 0.6 77.2) (end 1 76.5) (width 0.4) (layer "B.Cu") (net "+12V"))
 (segment (start 8.8 64.625) (end 9.7 64.625) (width 0.25) (layer "B.Cu") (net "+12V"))
 (segment (start 1 29.799999) (end 1.35 29.799999) (width 0.3) (layer "B.Cu") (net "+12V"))
 (segment (start 8.8 57.825) (end 9.7 57.825) (width 0.25) (layer "B.Cu") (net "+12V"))
 (segment (start 1 9.4) (end 1.35 9.4) (width 0.3) (layer "B.Cu") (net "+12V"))
 (segment (start 0.6 79.5) (end 0.6 77.2) (width 0.4) (layer "B.Cu") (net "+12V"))
 (segment (start 1 8.5) (end 9.7 8.5) (width 0.35) (layer "B.Cu") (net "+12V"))
 (segment (start 1 23) (end 1.35 23) (width 0.3) (layer "B.Cu") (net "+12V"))
 (segment (start 8.8 10.225) (end 9.7 10.225) (width 0.25) (layer "B.Cu") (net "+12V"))
 (segment (start 8.8 37.425) (end 9.7 37.425) (width 0.25) (layer "B.Cu") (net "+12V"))
 (segment (start 1 76.5) (end 1 8.5) (width 0.4) (layer "B.Cu") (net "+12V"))
 (segment (start 1 36.6) (end 1.35 36.6) (width 0.3) (layer "B.Cu") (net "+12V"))
 (segment (start 2.2 81.2) (end 0.6 79.5) (width 0.4) (layer "B.Cu") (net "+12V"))
 (segment (start 5.2 81.2) (end 5.225 82.5) (width 0.25) (layer "F.Cu") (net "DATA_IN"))
 (segment (start 3.3 12.6) (end 6.25 12.6) (width 0.25) (layer "F.Cu") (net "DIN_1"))
 (segment (start 3.3 12.6) (end 3.3 9.4) (width 0.25) (layer "F.Cu") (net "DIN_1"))
 (segment (start 3.3 9.4) (end 6.25 9.4) (width 0.25) (layer "F.Cu") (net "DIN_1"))
 (via (at 6.775 82.5) (size 0.6) (drill 0.3) (layers "F.Cu" "B.Cu") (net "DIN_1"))
 (via (at 3.3 12.6) (size 0.6) (drill 0.3) (layers "F.Cu" "B.Cu") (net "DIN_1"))
 (segment (start 3.3 79.5) (end 3.3 12.6) (width 0.22) (layer "B.Cu") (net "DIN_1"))
 (segment (start 3.7 82.5) (end 3.7 80.5) (width 0.22) (layer "B.Cu") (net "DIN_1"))
 (segment (start 3.7 80.5) (end 3.3 79.5) (width 0.22) (layer "B.Cu") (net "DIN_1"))
 (segment (start 6.775 82.5) (end 3.7 82.5) (width 0.22) (layer "B.Cu") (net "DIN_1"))
 (segment (start 1.35 73.8) (end 1.225 75.9) (width 0.25) (layer "F.Cu") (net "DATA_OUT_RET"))
 (segment (start 2.775 75.9) (end 2 78) (width 0.25) (layer "F.Cu") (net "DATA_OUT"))
 (segment (start 2.5 13.8) (end 3.8 14.4) (width 0.25) (layer "F.Cu") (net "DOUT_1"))
 (segment (start 3.8 16.2) (end 3.8 19.4) (width 0.25) (layer "F.Cu") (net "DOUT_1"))
 (segment (start 1.35 12.6) (end 2.5 13.8) (width 0.25) (layer "F.Cu") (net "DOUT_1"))
 (segment (start 3.8 19.4) (end 6.25 19.4) (width 0.25) (layer "F.Cu") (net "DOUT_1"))
 (segment (start 3.8 14.4) (end 3.8 16.2) (width 0.25) (layer "F.Cu") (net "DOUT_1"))
 (segment (start 3.8 16.2) (end 6.25 16.2) (width 0.25) (layer "F.Cu") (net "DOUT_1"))
 (segment (start 2.5 20.6) (end 3.8 21.2) (width 0.25) (layer "F.Cu") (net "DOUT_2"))
 (segment (start 3.8 26.2) (end 6.25 26.2) (width 0.25) (layer "F.Cu") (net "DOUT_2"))
 (segment (start 1.35 19.4) (end 2.5 20.6) (width 0.25) (layer "F.Cu") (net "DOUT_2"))
 (segment (start 3.8 23) (end 6.25 23) (width 0.25) (layer "F.Cu") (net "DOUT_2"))
 (segment (start 3.8 21.2) (end 3.8 23) (width 0.25) (layer "F.Cu") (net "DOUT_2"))
 (segment (start 3.8 23) (end 3.8 26.2) (width 0.25) (layer "F.Cu") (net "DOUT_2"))
 (segment (start 2.5 27.4) (end 3.8 28) (width 0.25) (layer "F.Cu") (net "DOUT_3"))
 (segment (start 1.35 26.2) (end 2.5 27.4) (width 0.25) (layer "F.Cu") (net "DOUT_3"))
 (segment (start 3.8 29.799999) (end 6.25 29.799999) (width 0.25) (layer "F.Cu") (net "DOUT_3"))
 (segment (start 3.8 28) (end 3.8 29.799999) (width 0.25) (layer "F.Cu") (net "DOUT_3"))
 (segment (start 3.8 33) (end 6.25 33) (width 0.25) (layer "F.Cu") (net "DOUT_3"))
 (segment (start 3.8 29.799999) (end 3.8 33) (width 0.25) (layer "F.Cu") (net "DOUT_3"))
 (segment (start 3.8 39.8) (end 6.25 39.8) (width 0.25) (layer "F.Cu") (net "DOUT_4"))
 (segment (start 3.8 34.8) (end 3.8 36.6) (width 0.25) (layer "F.Cu") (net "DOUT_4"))
 (segment (start 3.8 36.6) (end 3.8 39.8) (width 0.25) (layer "F.Cu") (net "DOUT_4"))
 (segment (start 3.8 36.6) (end 6.25 36.6) (width 0.25) (layer "F.Cu") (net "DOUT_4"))
 (segment (start 1.35 33) (end 2.5 34.199999) (width 0.25) (layer "F.Cu") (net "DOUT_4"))
 (segment (start 2.5 34.199999) (end 3.8 34.8) (width 0.25) (layer "F.Cu") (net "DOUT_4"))
 (segment (start 2.5 41) (end 3.8 41.6) (width 0.25) (layer "F.Cu") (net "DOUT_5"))
 (segment (start 3.8 43.4) (end 3.8 46.6) (width 0.25) (layer "F.Cu") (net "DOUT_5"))
 (segment (start 1.35 39.8) (end 2.5 41) (width 0.25) (layer "F.Cu") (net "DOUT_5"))
 (segment (start 3.8 43.4) (end 6.25 43.4) (width 0.25) (layer "F.Cu") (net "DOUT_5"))
 (segment (start 3.8 41.6) (end 3.8 43.4) (width 0.25) (layer "F.Cu") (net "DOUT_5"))
 (segment (start 3.8 46.6) (end 6.25 46.6) (width 0.25) (layer "F.Cu") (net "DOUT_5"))
 (segment (start 2.5 47.8) (end 3.8 48.4) (width 0.25) (layer "F.Cu") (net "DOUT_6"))
 (segment (start 3.8 48.4) (end 3.8 50.199999) (width 0.25) (layer "F.Cu") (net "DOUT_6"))
 (segment (start 3.8 53.4) (end 6.25 53.4) (width 0.25) (layer "F.Cu") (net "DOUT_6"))
 (segment (start 3.8 50.199999) (end 3.8 53.4) (width 0.25) (layer "F.Cu") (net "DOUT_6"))
 (segment (start 3.8 50.199999) (end 6.25 50.199999) (width 0.25) (layer "F.Cu") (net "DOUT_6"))
 (segment (start 1.35 46.6) (end 2.5 47.8) (width 0.25) (layer "F.Cu") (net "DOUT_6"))
 (segment (start 2.5 54.599999) (end 3.8 55.199999) (width 0.25) (layer "F.Cu") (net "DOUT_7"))
 (segment (start 3.8 57) (end 6.25 57) (width 0.25) (layer "F.Cu") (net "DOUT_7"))
 (segment (start 3.8 57) (end 3.8 60.2) (width 0.25) (layer "F.Cu") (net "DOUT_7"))
 (segment (start 1.35 53.4) (end 2.5 54.599999) (width 0.25) (layer "F.Cu") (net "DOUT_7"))
 (segment (start 3.8 60.2) (end 6.25 60.2) (width 0.25) (layer "F.Cu") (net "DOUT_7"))
 (segment (start 3.8 55.199999) (end 3.8 57) (width 0.25) (layer "F.Cu") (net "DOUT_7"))
 (segment (start 3.8 67) (end 6.25 67) (width 0.25) (layer "F.Cu") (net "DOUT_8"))
 (segment (start 3.8 63.8) (end 6.25 63.8) (width 0.25) (layer "F.Cu") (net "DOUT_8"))
 (segment (start 1.35 60.2) (end 2.5 61.4) (width 0.25) (layer "F.Cu") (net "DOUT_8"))
 (segment (start 2.5 61.4) (end 3.8 62) (width 0.25) (layer "F.Cu") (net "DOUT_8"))
 (segment (start 3.8 62) (end 3.8 63.8) (width 0.25) (layer "F.Cu") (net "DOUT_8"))
 (segment (start 3.8 63.8) (end 3.8 67) (width 0.25) (layer "F.Cu") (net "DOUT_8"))
 (segment (start 3.8 70.6) (end 3.8 73.799999) (width 0.25) (layer "F.Cu") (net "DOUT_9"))
 (segment (start 3.8 68.8) (end 3.8 70.6) (width 0.25) (layer "F.Cu") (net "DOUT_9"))
 (segment (start 3.8 73.799999) (end 6.25 73.799999) (width 0.25) (layer "F.Cu") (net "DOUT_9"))
 (segment (start 1.35 67) (end 2.5 68.2) (width 0.25) (layer "F.Cu") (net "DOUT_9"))
 (segment (start 3.8 70.6) (end 6.25 70.6) (width 0.25) (layer "F.Cu") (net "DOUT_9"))
 (segment (start 2.5 68.2) (end 3.8 68.8) (width 0.25) (layer "F.Cu") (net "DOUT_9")))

